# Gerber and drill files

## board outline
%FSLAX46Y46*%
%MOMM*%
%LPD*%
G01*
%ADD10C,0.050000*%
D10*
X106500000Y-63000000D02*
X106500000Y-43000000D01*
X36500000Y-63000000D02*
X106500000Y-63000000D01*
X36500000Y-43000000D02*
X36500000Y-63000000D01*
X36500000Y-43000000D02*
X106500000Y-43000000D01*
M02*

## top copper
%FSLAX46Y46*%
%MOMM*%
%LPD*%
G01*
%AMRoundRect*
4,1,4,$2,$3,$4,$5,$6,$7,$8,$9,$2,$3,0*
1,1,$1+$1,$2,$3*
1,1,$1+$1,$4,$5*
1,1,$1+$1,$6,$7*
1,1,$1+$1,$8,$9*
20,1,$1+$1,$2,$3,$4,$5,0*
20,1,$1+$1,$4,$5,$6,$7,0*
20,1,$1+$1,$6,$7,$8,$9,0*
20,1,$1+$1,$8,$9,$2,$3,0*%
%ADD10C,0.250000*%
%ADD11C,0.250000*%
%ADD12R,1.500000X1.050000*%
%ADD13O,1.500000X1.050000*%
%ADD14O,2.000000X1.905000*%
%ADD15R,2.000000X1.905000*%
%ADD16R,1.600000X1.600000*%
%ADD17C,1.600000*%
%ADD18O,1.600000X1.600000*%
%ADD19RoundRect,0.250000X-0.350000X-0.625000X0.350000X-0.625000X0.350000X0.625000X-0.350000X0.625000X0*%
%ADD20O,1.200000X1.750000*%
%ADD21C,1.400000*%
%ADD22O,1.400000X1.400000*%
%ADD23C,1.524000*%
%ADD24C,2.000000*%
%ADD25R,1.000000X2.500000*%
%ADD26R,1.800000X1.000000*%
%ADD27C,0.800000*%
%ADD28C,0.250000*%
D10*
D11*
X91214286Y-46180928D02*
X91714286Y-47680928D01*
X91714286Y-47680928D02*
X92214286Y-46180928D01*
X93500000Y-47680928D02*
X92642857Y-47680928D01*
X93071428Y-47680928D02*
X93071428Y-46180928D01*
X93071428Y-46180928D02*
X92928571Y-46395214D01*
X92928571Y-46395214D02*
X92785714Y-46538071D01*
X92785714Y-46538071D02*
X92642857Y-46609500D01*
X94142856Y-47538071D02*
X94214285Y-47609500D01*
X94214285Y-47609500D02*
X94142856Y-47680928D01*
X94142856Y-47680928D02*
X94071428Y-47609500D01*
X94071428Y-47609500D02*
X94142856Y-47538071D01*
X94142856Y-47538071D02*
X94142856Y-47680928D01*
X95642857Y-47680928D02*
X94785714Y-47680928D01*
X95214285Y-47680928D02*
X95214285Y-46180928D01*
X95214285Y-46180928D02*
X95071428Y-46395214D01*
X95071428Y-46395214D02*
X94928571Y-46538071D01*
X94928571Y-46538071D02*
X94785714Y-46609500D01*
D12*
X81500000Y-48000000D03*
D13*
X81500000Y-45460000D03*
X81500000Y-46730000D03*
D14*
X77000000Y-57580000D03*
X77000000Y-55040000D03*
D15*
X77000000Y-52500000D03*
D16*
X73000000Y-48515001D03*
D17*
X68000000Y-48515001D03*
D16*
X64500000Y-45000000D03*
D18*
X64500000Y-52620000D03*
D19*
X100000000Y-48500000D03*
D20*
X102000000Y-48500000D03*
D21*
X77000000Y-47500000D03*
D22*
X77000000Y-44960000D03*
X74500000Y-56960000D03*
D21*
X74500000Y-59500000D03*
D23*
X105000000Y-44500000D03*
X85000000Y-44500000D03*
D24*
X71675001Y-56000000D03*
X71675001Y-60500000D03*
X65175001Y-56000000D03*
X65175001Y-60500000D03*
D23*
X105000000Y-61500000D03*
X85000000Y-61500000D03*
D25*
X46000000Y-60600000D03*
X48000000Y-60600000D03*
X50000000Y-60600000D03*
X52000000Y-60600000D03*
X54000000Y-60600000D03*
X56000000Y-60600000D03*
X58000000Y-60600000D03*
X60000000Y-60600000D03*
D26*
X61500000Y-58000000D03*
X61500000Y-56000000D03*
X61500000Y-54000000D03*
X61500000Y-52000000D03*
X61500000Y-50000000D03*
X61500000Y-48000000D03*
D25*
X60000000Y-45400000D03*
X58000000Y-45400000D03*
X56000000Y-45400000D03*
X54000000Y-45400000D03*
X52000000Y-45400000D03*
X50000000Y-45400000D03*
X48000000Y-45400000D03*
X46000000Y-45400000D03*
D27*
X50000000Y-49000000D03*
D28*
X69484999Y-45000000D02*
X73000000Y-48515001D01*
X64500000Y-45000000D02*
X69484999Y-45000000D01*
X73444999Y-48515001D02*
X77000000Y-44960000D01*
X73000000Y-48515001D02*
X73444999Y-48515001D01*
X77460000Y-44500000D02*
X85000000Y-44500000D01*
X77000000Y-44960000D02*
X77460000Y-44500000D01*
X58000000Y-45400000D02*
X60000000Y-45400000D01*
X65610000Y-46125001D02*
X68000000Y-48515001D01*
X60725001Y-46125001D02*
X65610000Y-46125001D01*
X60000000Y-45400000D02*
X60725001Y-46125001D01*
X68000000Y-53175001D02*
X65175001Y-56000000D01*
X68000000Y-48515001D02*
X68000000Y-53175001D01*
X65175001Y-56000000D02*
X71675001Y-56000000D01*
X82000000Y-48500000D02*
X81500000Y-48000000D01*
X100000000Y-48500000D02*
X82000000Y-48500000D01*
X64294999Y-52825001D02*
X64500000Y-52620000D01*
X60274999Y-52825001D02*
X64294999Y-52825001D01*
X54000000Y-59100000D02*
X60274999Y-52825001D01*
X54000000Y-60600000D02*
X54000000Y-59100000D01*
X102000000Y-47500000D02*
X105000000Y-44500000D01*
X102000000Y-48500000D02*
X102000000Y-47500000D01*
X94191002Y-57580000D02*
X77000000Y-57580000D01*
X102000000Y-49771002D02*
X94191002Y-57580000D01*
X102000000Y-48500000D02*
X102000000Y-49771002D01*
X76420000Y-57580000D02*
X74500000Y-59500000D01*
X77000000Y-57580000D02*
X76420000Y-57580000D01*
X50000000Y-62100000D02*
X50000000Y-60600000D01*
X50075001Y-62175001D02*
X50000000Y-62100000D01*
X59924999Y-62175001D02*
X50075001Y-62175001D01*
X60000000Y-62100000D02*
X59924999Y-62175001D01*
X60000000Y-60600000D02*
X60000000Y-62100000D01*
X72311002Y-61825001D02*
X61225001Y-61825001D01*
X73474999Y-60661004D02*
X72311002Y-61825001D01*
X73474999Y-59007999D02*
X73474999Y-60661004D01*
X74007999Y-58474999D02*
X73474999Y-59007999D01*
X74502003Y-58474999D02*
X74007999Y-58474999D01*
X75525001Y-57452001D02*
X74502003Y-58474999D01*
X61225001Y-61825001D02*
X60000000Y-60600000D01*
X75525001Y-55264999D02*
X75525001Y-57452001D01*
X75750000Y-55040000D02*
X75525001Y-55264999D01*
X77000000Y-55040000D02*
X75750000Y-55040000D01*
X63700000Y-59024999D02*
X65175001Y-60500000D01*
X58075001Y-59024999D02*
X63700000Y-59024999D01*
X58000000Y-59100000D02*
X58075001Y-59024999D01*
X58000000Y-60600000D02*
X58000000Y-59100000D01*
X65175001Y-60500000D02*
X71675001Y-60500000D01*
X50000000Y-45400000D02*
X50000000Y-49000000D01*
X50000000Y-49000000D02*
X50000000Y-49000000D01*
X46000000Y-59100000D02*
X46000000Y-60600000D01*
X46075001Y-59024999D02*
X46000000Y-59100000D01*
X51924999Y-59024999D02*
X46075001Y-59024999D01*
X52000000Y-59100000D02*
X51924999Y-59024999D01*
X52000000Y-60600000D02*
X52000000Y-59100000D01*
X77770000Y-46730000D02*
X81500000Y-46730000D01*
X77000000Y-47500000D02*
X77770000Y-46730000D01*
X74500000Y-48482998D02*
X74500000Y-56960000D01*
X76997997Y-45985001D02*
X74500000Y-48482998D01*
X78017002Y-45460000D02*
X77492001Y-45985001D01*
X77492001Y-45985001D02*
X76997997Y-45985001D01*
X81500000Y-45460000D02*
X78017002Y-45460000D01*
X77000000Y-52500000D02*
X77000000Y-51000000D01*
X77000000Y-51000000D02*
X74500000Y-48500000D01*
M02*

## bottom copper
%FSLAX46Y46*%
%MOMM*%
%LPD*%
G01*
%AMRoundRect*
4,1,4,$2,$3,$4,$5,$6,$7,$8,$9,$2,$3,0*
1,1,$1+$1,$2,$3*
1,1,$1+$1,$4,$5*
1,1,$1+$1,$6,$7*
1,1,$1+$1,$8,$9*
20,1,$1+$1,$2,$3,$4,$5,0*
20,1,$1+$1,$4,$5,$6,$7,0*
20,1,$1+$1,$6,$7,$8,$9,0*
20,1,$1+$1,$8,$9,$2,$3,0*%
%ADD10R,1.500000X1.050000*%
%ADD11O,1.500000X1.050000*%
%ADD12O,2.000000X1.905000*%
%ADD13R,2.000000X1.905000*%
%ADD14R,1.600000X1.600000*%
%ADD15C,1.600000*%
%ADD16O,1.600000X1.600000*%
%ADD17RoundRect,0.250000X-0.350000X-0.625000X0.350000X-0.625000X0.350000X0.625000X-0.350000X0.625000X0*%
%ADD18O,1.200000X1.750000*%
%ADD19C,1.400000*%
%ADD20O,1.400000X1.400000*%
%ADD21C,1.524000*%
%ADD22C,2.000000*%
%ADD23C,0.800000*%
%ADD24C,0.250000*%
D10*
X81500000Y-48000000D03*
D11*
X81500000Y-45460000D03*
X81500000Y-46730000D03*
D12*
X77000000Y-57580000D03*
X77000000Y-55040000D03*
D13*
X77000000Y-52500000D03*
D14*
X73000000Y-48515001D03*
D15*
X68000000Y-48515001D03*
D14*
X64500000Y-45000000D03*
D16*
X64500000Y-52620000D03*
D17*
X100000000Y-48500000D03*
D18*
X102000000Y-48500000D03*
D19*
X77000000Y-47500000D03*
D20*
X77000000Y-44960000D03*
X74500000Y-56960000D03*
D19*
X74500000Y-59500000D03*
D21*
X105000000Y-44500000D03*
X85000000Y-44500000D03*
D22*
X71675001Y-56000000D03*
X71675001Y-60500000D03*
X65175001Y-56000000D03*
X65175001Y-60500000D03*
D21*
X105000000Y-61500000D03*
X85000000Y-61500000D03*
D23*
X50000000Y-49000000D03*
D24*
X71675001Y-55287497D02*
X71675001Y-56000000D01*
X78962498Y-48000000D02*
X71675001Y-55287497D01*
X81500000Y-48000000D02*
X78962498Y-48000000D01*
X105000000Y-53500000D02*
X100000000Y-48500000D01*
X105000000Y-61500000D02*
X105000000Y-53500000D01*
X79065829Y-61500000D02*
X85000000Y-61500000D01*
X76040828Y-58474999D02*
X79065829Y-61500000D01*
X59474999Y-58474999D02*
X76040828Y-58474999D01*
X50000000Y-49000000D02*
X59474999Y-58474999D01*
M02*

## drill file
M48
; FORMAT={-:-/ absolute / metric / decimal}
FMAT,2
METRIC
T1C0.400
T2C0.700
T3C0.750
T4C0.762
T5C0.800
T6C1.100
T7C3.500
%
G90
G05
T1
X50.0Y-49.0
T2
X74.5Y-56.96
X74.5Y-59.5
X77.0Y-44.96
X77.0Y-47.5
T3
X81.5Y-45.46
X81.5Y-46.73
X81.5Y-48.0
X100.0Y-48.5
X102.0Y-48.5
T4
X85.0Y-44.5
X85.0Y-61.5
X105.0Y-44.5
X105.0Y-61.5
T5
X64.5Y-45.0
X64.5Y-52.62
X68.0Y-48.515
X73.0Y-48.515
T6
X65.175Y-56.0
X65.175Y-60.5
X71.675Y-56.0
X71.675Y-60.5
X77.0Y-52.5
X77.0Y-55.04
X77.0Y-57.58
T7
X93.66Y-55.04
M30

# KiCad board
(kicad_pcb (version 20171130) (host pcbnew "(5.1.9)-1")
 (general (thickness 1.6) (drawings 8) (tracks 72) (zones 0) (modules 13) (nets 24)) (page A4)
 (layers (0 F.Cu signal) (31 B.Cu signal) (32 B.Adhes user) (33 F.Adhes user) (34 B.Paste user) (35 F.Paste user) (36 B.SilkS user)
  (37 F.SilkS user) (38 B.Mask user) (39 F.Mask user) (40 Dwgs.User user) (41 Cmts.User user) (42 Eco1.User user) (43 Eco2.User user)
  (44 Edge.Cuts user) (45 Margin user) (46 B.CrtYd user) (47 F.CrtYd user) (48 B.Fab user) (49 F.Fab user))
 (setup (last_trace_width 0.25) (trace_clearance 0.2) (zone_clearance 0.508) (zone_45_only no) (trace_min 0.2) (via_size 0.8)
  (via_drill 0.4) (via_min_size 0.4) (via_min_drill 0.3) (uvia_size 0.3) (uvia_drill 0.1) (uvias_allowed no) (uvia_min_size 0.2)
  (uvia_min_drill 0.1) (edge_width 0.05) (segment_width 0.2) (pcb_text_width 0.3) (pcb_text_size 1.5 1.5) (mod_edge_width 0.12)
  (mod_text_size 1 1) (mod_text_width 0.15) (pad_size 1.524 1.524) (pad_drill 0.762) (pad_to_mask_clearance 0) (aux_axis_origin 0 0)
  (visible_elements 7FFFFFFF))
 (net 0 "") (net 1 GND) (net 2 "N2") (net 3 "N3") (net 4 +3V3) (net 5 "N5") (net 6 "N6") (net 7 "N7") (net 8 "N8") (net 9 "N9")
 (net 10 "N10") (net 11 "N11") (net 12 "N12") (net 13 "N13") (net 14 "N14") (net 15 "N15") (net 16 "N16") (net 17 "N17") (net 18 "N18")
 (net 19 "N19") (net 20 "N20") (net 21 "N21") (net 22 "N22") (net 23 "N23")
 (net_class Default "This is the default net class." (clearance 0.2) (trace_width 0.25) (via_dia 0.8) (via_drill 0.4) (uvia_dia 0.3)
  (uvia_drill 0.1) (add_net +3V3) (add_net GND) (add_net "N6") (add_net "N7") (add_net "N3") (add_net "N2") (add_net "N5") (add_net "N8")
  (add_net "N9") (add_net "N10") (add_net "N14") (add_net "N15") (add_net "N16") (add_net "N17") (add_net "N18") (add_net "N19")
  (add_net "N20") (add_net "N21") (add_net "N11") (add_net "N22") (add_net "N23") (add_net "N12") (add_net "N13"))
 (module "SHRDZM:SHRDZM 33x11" (layer B.Cu) (at 54 50.5 180)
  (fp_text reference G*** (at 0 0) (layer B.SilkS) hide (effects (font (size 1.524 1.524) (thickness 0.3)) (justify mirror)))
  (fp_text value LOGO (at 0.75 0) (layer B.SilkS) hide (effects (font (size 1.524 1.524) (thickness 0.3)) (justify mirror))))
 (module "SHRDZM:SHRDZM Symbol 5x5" (layer F.Cu) (at 101 59.5)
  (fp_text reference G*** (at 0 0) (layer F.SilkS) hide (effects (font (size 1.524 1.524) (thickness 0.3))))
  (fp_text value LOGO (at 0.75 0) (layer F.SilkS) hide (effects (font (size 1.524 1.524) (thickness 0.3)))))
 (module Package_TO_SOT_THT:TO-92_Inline (layer F.Cu) (at 81.5 48 90)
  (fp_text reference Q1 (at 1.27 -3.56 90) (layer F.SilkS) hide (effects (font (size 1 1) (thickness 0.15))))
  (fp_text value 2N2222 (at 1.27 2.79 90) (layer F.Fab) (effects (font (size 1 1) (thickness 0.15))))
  (pad 1 thru_hole rect (at 0 0 90) (size 1.05 1.5) (drill 0.75) (layers *.Cu *.Mask) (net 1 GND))
  (pad 3 thru_hole oval (at 2.54 0 90) (size 1.05 1.5) (drill 0.75) (layers *.Cu *.Mask) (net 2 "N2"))
  (pad 2 thru_hole oval (at 1.27 0 90) (size 1.05 1.5) (drill 0.75) (layers *.Cu *.Mask) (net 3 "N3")))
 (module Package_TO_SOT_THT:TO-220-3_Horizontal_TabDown (layer F.Cu) (at 77 52.5 270)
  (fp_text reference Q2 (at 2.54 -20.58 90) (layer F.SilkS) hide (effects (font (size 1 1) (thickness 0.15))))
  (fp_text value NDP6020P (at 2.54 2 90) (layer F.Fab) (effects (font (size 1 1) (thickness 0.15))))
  (pad 3 thru_hole oval (at 5.08 0 270) (size 1.905 2) (drill 1.1) (layers *.Cu *.Mask) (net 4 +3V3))
  (pad 2 thru_hole oval (at 2.54 0 270) (size 1.905 2) (drill 1.1) (layers *.Cu *.Mask) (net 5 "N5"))
  (pad 1 thru_hole rect (at 0 0 270) (size 1.905 2) (drill 1.1) (layers *.Cu *.Mask) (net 2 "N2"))
  (pad "" np_thru_hole oval (at 2.54 -16.66 270) (size 3.5 3.5) (drill 3.5) (layers *.Cu *.Mask)))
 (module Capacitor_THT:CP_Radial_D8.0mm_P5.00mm (layer F.Cu) (at 73 48.515001 180)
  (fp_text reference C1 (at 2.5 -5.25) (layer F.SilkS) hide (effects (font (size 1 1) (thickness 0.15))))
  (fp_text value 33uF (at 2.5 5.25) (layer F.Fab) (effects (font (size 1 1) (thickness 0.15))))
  (pad 1 thru_hole rect (at 0 0 180) (size 1.6 1.6) (drill 0.8) (layers *.Cu *.Mask) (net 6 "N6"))
  (pad 2 thru_hole circle (at 5 0 180) (size 1.6 1.6) (drill 0.8) (layers *.Cu *.Mask) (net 1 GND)))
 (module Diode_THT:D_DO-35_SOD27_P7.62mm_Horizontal (layer F.Cu) (at 64.5 45 270)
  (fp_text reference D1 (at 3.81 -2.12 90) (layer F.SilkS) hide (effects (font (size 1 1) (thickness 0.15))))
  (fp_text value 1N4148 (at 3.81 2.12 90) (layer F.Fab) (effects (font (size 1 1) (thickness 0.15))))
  (pad 1 thru_hole rect (at 0 0 270) (size 1.6 1.6) (drill 0.8) (layers *.Cu *.Mask) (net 6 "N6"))
  (pad 2 thru_hole oval (at 7.62 0 270) (size 1.6 1.6) (drill 0.8) (layers *.Cu *.Mask) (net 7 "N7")))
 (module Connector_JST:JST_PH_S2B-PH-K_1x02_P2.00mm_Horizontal (layer F.Cu) (at 100 48.5)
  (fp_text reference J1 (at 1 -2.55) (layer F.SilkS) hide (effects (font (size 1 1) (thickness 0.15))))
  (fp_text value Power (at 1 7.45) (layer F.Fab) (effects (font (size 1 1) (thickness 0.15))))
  (pad 1 thru_hole roundrect (at 0 0) (size 1.2 1.75) (drill 0.75) (layers *.Cu *.Mask) (roundrect_rratio 0.208333) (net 1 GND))
  (pad 2 thru_hole oval (at 2 0) (size 1.2 1.75) (drill 0.75) (layers *.Cu *.Mask) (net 4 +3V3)))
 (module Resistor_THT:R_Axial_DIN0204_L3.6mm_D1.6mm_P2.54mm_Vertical (layer F.Cu) (at 77 47.5 90)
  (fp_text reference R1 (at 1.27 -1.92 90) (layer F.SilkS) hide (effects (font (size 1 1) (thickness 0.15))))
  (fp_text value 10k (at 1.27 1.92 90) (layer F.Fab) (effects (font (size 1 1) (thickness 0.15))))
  (pad 1 thru_hole circle (at 0 0 90) (size 1.4 1.4) (drill 0.7) (layers *.Cu *.Mask) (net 3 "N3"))
  (pad 2 thru_hole oval (at 2.54 0 90) (size 1.4 1.4) (drill 0.7) (layers *.Cu *.Mask) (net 6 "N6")))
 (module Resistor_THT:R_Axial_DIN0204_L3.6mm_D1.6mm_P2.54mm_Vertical (layer F.Cu) (at 74.5 59.5 90)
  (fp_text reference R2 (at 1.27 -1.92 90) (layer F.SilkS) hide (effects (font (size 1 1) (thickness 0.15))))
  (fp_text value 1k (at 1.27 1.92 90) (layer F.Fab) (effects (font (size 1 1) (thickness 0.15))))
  (pad 2 thru_hole oval (at 2.54 0 90) (size 1.4 1.4) (drill 0.7) (layers *.Cu *.Mask) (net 2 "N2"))
  (pad 1 thru_hole circle (at 0 0 90) (size 1.4 1.4) (drill 0.7) (layers *.Cu *.Mask) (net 4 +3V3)))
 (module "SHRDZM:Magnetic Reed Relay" (layer F.Cu) (at 95 44.5 180)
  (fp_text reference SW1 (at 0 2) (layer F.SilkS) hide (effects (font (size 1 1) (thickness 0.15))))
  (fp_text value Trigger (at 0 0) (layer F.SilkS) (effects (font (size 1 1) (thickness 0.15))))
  (pad 1 thru_hole circle (at -10 0 180) (size 1.524 1.524) (drill 0.762) (layers *.Cu *.Mask) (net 4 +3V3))
  (pad 2 thru_hole circle (at 10 0 180) (size 1.524 1.524) (drill 0.762) (layers *.Cu *.Mask) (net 6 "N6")))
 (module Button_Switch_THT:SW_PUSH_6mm (layer F.Cu) (at 71.675001 60.5 180)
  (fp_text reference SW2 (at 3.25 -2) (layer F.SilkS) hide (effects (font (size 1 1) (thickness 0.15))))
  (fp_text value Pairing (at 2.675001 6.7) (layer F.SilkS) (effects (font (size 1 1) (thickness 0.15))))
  (pad 2 thru_hole circle (at 0 4.5 270) (size 2 2) (drill 1.1) (layers *.Cu *.Mask) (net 1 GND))
  (pad 1 thru_hole circle (at 0 0 270) (size 2 2) (drill 1.1) (layers *.Cu *.Mask) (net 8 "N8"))
  (pad 2 thru_hole circle (at 6.5 4.5 270) (size 2 2) (drill 1.1) (layers *.Cu *.Mask) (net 1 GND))
  (pad 1 thru_hole circle (at 6.5 0 270) (size 2 2) (drill 1.1) (layers *.Cu *.Mask) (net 8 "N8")))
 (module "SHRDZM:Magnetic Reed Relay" (layer B.Cu) (at 95 61.5)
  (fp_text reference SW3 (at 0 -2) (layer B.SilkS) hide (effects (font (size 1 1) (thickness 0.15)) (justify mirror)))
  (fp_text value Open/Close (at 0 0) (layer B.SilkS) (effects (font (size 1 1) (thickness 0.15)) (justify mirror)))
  (pad 2 thru_hole circle (at 10 0) (size 1.524 1.524) (drill 0.762) (layers *.Cu *.Mask) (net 1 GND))
  (pad 1 thru_hole circle (at -10 0) (size 1.524 1.524) (drill 0.762) (layers *.Cu *.Mask) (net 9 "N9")))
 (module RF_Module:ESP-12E (layer F.Cu) (at 49.5 53 90)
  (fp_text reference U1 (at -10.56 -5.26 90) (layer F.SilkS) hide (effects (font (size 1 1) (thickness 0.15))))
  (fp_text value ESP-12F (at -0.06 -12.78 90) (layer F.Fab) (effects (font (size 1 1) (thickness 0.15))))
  (pad 1 smd rect (at -7.6 -3.5 90) (size 2.5 1) (layers F.Cu F.Paste F.Mask) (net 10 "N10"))
  (pad 2 smd rect (at -7.6 -1.5 90) (size 2.5 1) (layers F.Cu F.Paste F.Mask) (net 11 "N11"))
  (pad 3 smd rect (at -7.6 0.5 90) (size 2.5 1) (layers F.Cu F.Paste F.Mask) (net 5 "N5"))
  (pad 4 smd rect (at -7.6 2.5 90) (size 2.5 1) (layers F.Cu F.Paste F.Mask) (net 10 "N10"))
  (pad 5 smd rect (at -7.6 4.5 90) (size 2.5 1) (layers F.Cu F.Paste F.Mask) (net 7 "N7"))
  (pad 6 smd rect (at -7.6 6.5 90) (size 2.5 1) (layers F.Cu F.Paste F.Mask) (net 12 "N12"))
  (pad 7 smd rect (at -7.6 8.5 90) (size 2.5 1) (layers F.Cu F.Paste F.Mask) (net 8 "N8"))
  (pad 8 smd rect (at -7.6 10.5 90) (size 2.5 1) (layers F.Cu F.Paste F.Mask) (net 5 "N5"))
  (pad 9 smd rect (at -5 12 90) (size 1 1.8) (layers F.Cu F.Paste F.Mask) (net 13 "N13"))
  (pad 10 smd rect (at -3 12 90) (size 1 1.8) (layers F.Cu F.Paste F.Mask) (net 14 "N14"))
  (pad 11 smd rect (at -1 12 90) (size 1 1.8) (layers F.Cu F.Paste F.Mask) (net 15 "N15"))
  (pad 12 smd rect (at 1 12 90) (size 1 1.8) (layers F.Cu F.Paste F.Mask) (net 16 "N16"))
  (pad 13 smd rect (at 3 12 90) (size 1 1.8) (layers F.Cu F.Paste F.Mask) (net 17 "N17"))
  (pad 14 smd rect (at 5 12 90) (size 1 1.8) (layers F.Cu F.Paste F.Mask) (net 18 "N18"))
  (pad 15 smd rect (at 7.6 10.5 90) (size 2.5 1) (layers F.Cu F.Paste F.Mask) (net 1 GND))
  (pad 16 smd rect (at 7.6 8.5 90) (size 2.5 1) (layers F.Cu F.Paste F.Mask) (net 1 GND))
  (pad 17 smd rect (at 7.6 6.5 90) (size 2.5 1) (layers F.Cu F.Paste F.Mask) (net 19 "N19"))
  (pad 18 smd rect (at 7.6 4.5 90) (size 2.5 1) (layers F.Cu F.Paste F.Mask) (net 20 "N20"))
  (pad 19 smd rect (at 7.6 2.5 90) (size 2.5 1) (layers F.Cu F.Paste F.Mask) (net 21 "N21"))
  (pad 20 smd rect (at 7.6 0.5 90) (size 2.5 1) (layers F.Cu F.Paste F.Mask) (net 9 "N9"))
  (pad 21 smd rect (at 7.6 -1.5 90) (size 2.5 1) (layers F.Cu F.Paste F.Mask) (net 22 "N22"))
  (pad 22 smd rect (at 7.6 -3.5 90) (size 2.5 1) (layers F.Cu F.Paste F.Mask) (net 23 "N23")))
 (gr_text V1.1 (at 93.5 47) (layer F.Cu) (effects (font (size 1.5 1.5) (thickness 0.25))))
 (gr_line (start 106.5 63) (end 106.5 43) (layer Edge.Cuts) (width 0.05))
 (gr_line (start 36.5 63) (end 106.5 63) (layer Edge.Cuts) (width 0.05))
 (gr_line (start 36.5 43) (end 36.5 63) (layer Edge.Cuts) (width 0.05))
 (gr_line (start 36.5 43) (end 106.5 43) (layer Edge.Cuts) (width 0.05))
 (segment (start 69.484999 45) (end 73 48.515001) (width 0.25) (layer F.Cu) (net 6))
 (segment (start 64.5 45) (end 69.484999 45) (width 0.25) (layer F.Cu) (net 6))
 (segment (start 73.444999 48.515001) (end 77 44.96) (width 0.25) (layer F.Cu) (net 6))
 (segment (start 73 48.515001) (end 73.444999 48.515001) (width 0.25) (layer F.Cu) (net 6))
 (segment (start 77.46 44.5) (end 85 44.5) (width 0.25) (layer F.Cu) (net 6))
 (segment (start 77 44.96) (end 77.46 44.5) (width 0.25) (layer F.Cu) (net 6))
 (segment (start 58 45.4) (end 60 45.4) (width 0.25) (layer F.Cu) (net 1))
 (segment (start 65.61 46.125001) (end 68 48.515001) (width 0.25) (layer F.Cu) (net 1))
 (segment (start 60.725001 46.125001) (end 65.61 46.125001) (width 0.25) (layer F.Cu) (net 1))
 (segment (start 60 45.4) (end 60.725001 46.125001) (width 0.25) (layer F.Cu) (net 1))
 (segment (start 68 53.175001) (end 65.175001 56) (width 0.25) (layer F.Cu) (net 1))
 (segment (start 68 48.515001) (end 68 53.175001) (width 0.25) (layer F.Cu) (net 1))
 (segment (start 65.175001 56) (end 71.675001 56) (width 0.25) (layer F.Cu) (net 1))
 (segment (start 71.675001 55.287497) (end 71.675001 56) (width 0.25) (layer B.Cu) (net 1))
 (segment (start 78.962498 48) (end 71.675001 55.287497) (width 0.25) (layer B.Cu) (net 1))
 (segment (start 81.5 48) (end 78.962498 48) (width 0.25) (layer B.Cu) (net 1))
 (segment (start 82 48.5) (end 81.5 48) (width 0.25) (layer F.Cu) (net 1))
 (segment (start 100 48.5) (end 82 48.5) (width 0.25) (layer F.Cu) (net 1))
 (segment (start 105 53.5) (end 100 48.5) (width 0.25) (layer B.Cu) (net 1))
 (segment (start 105 61.5) (end 105 53.5) (width 0.25) (layer B.Cu) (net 1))
 (segment (start 64.294999 52.825001) (end 64.5 52.62) (width 0.25) (layer F.Cu) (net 7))
 (segment (start 60.274999 52.825001) (end 64.294999 52.825001) (width 0.25) (layer F.Cu) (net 7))
 (segment (start 54 59.1) (end 60.274999 52.825001) (width 0.25) (layer F.Cu) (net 7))
 (segment (start 54 60.6) (end 54 59.1) (width 0.25) (layer F.Cu) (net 7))
 (segment (start 102 47.5) (end 105 44.5) (width 0.25) (layer F.Cu) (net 4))
 (segment (start 102 48.5) (end 102 47.5) (width 0.25) (layer F.Cu) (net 4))
 (segment (start 94.191002 57.58) (end 77 57.58) (width 0.25) (layer F.Cu) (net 4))
 (segment (start 102 49.771002) (end 94.191002 57.58) (width 0.25) (layer F.Cu) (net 4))
 (segment (start 102 48.5) (end 102 49.771002) (width 0.25) (layer F.Cu) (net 4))
 (segment (start 76.42 57.58) (end 74.5 59.5) (width 0.25) (layer F.Cu) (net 4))
 (segment (start 77 57.58) (end 76.42 57.58) (width 0.25) (layer F.Cu) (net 4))
 (segment (start 50 62.1) (end 50 60.6) (width 0.25) (layer F.Cu) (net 5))
 (segment (start 50.075001 62.175001) (end 50 62.1) (width 0.25) (layer F.Cu) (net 5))
 (segment (start 59.924999 62.175001) (end 50.075001 62.175001) (width 0.25) (layer F.Cu) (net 5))
 (segment (start 60 62.1) (end 59.924999 62.175001) (width 0.25) (layer F.Cu) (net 5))
 (segment (start 60 60.6) (end 60 62.1) (width 0.25) (layer F.Cu) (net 5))
 (segment (start 72.311002 61.825001) (end 61.225001 61.825001) (width 0.25) (layer F.Cu) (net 5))
 (segment (start 73.474999 60.661004) (end 72.311002 61.825001) (width 0.25) (layer F.Cu) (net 5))
 (segment (start 73.474999 59.007999) (end 73.474999 60.661004) (width 0.25) (layer F.Cu) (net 5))
 (segment (start 74.007999 58.474999) (end 73.474999 59.007999) (width 0.25) (layer F.Cu) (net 5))
 (segment (start 74.502003 58.474999) (end 74.007999 58.474999) (width 0.25) (layer F.Cu) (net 5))
 (segment (start 75.525001 57.452001) (end 74.502003 58.474999) (width 0.25) (layer F.Cu) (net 5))
 (segment (start 61.225001 61.825001) (end 60 60.6) (width 0.25) (layer F.Cu) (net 5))
 (segment (start 75.525001 55.264999) (end 75.525001 57.452001) (width 0.25) (layer F.Cu) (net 5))
 (segment (start 75.75 55.04) (end 75.525001 55.264999) (width 0.25) (layer F.Cu) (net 5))
 (segment (start 77 55.04) (end 75.75 55.04) (width 0.25) (layer F.Cu) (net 5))
 (segment (start 63.7 59.024999) (end 65.175001 60.5) (width 0.25) (layer F.Cu) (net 8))
 (segment (start 58.075001 59.024999) (end 63.7 59.024999) (width 0.25) (layer F.Cu) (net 8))
 (segment (start 58 59.1) (end 58.075001 59.024999) (width 0.25) (layer F.Cu) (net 8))
 (segment (start 58 60.6) (end 58 59.1) (width 0.25) (layer F.Cu) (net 8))
 (segment (start 65.175001 60.5) (end 71.675001 60.5) (width 0.25) (layer F.Cu) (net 8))
 (segment (start 50 45.4) (end 50 49) (width 0.25) (layer F.Cu) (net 9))
 (segment (start 50 49) (end 50 49) (width 0.25) (layer F.Cu) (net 9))
 (via (at 50 49) (size 0.8) (drill 0.4) (layers F.Cu B.Cu) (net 9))
 (segment (start 79.065829 61.5) (end 85 61.5) (width 0.25) (layer B.Cu) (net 9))
 (segment (start 76.040828 58.474999) (end 79.065829 61.5) (width 0.25) (layer B.Cu) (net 9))
 (segment (start 59.474999 58.474999) (end 76.040828 58.474999) (width 0.25) (layer B.Cu) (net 9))
 (segment (start 50 49) (end 59.474999 58.474999) (width 0.25) (layer B.Cu) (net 9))
 (segment (start 46 59.1) (end 46 60.6) (width 0.25) (layer F.Cu) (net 10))
 (segment (start 46.075001 59.024999) (end 46 59.1) (width 0.25) (layer F.Cu) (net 10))
 (segment (start 51.924999 59.024999) (end 46.075001 59.024999) (width 0.25) (layer F.Cu) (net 10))
 (segment (start 52 59.1) (end 51.924999 59.024999) (width 0.25) (layer F.Cu) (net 10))
 (segment (start 52 60.6) (end 52 59.1) (width 0.25) (layer F.Cu) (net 10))
 (segment (start 77.77 46.73) (end 81.5 46.73) (width 0.25) (layer F.Cu) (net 3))
 (segment (start 77 47.5) (end 77.77 46.73) (width 0.25) (layer F.Cu) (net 3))
 (segment (start 74.5 48.482998) (end 74.5 56.96) (width 0.25) (layer F.Cu) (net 2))
 (segment (start 76.997997 45.985001) (end 74.5 48.482998) (width 0.25) (layer F.Cu) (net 2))
 (segment (start 78.017002 45.46) (end 77.492001 45.985001) (width 0.25) (layer F.Cu) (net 2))
 (segment (start 77.492001 45.985001) (end 76.997997 45.985001) (width 0.25) (layer F.Cu) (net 2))
 (segment (start 81.5 45.46) (end 78.017002 45.46) (width 0.25) (layer F.Cu) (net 2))
 (segment (start 77 52.5) (end 77 51) (width 0.25) (layer F.Cu) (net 2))
 (segment (start 77 51) (end 74.5 48.5) (width 0.25) (layer F.Cu) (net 2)))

